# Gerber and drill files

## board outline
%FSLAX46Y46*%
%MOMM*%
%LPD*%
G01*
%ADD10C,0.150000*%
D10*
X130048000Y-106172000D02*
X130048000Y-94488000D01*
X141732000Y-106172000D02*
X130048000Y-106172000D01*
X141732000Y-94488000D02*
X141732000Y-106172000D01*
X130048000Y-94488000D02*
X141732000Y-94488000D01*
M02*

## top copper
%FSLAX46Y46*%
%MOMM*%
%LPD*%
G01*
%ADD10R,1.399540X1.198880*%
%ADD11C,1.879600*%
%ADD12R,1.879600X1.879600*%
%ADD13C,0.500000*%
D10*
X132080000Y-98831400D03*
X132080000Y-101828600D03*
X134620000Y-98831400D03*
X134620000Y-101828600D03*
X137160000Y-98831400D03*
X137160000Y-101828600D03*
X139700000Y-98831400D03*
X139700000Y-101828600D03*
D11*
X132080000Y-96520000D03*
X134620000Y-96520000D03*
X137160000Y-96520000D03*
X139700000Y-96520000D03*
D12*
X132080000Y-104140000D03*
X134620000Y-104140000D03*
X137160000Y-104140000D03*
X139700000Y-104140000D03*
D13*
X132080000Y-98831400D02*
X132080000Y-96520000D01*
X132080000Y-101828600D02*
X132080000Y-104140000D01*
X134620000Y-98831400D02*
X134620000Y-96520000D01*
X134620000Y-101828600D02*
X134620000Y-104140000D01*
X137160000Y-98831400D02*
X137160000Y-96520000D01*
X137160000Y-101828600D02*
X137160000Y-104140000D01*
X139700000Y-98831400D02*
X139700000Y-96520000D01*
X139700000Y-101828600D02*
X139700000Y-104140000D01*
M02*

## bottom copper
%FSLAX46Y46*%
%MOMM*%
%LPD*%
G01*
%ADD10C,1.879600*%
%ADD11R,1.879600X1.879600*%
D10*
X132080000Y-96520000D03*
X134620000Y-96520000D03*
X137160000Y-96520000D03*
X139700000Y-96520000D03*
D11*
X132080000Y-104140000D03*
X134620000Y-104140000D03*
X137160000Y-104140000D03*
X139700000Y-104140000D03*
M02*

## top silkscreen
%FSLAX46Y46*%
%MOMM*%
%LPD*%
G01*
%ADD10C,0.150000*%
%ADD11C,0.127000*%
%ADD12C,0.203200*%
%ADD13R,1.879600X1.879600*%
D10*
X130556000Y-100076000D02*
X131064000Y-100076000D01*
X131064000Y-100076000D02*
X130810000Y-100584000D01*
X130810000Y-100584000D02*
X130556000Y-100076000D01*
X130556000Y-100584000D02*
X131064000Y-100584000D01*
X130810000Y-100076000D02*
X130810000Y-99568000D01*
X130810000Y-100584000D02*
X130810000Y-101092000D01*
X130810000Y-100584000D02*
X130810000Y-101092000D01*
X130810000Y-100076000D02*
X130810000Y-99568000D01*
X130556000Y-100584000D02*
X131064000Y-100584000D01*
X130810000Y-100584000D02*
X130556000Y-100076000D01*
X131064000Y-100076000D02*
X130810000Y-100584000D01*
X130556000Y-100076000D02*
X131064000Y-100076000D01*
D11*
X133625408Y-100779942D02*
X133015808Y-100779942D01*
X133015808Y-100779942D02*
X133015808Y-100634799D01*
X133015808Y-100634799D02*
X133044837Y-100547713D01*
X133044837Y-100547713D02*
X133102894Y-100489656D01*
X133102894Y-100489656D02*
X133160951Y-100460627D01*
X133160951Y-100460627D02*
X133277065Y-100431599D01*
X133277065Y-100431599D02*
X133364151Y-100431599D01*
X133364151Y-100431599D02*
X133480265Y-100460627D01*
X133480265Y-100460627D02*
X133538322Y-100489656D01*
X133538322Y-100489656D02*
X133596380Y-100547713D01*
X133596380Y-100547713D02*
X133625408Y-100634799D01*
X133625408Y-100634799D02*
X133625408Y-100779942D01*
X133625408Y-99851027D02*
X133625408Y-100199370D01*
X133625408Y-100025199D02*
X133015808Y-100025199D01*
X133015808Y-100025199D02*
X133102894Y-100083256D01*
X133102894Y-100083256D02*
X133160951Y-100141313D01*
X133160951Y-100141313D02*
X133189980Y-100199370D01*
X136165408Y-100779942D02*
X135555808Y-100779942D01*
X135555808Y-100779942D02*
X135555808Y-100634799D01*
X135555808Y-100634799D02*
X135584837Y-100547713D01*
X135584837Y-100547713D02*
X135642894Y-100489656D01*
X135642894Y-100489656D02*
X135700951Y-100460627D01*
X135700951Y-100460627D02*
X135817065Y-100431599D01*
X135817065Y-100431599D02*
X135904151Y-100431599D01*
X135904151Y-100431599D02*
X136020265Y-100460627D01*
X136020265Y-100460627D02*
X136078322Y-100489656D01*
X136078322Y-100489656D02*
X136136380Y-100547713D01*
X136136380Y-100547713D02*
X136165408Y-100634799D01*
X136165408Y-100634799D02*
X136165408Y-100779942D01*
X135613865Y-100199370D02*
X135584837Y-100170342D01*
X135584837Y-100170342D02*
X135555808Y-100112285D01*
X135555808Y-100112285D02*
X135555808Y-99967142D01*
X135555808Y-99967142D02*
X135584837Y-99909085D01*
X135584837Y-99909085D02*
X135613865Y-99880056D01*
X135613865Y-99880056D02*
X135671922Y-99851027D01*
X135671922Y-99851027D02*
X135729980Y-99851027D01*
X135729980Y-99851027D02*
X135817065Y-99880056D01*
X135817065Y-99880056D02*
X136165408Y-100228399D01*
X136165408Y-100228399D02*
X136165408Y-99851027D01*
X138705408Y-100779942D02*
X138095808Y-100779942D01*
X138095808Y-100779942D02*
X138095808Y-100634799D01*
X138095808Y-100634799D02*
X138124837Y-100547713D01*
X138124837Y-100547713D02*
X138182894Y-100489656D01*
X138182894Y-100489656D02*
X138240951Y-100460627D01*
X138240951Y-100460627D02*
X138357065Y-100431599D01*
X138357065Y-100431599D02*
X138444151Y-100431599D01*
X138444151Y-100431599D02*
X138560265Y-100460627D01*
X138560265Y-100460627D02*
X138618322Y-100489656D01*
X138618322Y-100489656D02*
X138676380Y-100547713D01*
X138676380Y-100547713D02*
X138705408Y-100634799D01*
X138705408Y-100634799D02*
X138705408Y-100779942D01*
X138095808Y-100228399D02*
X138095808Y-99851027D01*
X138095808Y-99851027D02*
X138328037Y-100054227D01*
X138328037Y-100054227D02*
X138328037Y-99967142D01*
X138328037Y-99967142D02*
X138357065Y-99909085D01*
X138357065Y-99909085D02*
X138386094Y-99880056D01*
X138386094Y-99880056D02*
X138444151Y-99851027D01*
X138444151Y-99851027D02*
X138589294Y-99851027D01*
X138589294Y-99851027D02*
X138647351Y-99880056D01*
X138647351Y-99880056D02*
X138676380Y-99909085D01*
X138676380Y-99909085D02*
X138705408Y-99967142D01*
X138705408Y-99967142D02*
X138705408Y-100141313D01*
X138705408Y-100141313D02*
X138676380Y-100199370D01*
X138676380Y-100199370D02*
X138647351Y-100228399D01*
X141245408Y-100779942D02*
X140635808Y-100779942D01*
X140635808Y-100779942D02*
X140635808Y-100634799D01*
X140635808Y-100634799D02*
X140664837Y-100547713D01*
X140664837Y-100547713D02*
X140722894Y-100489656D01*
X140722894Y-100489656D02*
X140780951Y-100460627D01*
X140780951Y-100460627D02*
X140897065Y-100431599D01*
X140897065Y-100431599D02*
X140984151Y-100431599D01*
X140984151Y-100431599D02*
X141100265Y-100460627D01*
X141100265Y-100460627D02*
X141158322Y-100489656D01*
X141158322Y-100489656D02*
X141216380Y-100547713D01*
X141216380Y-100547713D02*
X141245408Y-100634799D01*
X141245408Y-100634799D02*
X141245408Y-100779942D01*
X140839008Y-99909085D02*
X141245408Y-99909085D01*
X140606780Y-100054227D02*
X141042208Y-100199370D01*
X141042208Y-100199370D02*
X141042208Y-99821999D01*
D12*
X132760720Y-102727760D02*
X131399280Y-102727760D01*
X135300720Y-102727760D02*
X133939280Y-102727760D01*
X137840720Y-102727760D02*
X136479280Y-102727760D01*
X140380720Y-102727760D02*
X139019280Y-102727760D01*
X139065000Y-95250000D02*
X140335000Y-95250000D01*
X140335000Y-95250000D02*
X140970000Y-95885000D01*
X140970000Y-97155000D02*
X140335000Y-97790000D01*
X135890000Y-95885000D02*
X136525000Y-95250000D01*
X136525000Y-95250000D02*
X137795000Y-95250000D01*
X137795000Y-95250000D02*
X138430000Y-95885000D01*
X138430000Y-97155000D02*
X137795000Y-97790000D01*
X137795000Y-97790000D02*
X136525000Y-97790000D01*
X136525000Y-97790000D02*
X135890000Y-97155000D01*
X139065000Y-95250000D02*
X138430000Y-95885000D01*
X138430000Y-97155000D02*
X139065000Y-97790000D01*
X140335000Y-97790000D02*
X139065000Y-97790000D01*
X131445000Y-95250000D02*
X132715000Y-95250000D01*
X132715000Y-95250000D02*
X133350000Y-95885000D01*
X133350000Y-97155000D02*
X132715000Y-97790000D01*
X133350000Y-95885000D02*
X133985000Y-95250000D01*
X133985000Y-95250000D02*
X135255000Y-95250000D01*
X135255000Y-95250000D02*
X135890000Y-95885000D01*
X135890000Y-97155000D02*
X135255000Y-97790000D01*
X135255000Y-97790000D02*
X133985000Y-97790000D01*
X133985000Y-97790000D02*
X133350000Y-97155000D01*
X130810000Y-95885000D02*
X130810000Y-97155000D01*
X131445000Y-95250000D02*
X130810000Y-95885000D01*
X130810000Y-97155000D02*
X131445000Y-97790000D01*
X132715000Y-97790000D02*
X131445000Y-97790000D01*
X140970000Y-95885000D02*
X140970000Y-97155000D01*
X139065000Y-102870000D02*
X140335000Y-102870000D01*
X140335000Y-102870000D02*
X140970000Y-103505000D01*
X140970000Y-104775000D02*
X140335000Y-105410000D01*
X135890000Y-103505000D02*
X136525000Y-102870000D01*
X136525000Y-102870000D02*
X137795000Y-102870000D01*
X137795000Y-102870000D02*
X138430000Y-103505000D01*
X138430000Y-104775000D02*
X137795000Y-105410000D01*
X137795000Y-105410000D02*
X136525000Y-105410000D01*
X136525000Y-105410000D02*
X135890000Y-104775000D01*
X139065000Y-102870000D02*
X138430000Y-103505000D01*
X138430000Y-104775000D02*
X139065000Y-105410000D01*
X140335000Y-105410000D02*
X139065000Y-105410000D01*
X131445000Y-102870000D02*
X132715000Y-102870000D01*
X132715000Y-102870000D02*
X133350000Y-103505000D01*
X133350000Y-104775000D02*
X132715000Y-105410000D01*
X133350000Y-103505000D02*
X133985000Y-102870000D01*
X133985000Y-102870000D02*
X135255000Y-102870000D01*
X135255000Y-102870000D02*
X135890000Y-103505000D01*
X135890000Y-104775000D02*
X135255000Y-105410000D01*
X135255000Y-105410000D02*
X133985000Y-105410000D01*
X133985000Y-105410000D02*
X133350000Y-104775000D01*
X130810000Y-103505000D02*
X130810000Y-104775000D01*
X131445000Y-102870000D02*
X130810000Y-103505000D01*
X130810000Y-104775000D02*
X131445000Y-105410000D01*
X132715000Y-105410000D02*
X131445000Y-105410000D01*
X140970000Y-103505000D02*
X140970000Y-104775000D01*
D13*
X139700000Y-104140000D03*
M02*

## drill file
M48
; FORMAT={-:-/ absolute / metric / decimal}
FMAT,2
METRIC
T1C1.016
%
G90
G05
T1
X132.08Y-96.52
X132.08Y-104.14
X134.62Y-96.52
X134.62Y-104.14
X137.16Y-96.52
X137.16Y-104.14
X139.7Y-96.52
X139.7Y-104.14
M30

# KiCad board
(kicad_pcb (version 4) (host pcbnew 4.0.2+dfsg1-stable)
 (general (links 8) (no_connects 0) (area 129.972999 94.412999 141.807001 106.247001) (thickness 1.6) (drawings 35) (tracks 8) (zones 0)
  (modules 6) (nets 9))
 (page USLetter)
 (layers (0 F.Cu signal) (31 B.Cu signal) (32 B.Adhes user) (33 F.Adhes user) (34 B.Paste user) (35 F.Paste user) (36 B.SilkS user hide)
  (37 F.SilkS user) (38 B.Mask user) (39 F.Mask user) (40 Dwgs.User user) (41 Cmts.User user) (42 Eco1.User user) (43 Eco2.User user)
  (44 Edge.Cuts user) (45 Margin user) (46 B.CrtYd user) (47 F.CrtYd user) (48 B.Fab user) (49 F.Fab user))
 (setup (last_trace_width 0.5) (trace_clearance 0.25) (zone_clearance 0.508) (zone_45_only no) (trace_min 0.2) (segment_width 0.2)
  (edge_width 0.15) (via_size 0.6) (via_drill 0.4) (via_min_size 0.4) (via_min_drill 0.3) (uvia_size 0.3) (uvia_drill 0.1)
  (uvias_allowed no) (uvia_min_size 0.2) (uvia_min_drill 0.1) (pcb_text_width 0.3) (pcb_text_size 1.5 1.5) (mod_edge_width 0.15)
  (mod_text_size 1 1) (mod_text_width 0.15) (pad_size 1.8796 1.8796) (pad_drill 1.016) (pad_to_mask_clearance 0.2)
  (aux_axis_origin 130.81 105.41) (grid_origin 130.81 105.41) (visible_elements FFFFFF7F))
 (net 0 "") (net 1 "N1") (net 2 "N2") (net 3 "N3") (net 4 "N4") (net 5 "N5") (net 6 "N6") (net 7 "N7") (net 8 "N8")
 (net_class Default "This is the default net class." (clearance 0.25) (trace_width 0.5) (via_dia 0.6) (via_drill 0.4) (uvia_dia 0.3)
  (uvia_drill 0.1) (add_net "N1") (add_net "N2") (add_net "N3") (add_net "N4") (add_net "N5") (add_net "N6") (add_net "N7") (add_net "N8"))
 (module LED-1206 (layer F.Cu) (at 132.08 100.33 270)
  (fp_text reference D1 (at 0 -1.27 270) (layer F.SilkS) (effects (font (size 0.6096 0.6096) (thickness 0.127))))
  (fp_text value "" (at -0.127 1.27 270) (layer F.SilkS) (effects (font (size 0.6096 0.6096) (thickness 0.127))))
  (fp_line (start 2.39776 -0.68072) (end 2.39776 0.68072) (layer F.SilkS) (width 0.2032))
  (pad A smd rect (at -1.4986 0 270) (size 1.19888 1.39954) (layers F.Cu F.Paste F.Mask) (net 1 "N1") (solder_mask_margin 0.1016))
  (pad C smd rect (at 1.4986 0 270) (size 1.19888 1.39954) (layers F.Cu F.Paste F.Mask) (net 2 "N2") (solder_mask_margin 0.1016)))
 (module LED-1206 (layer F.Cu) (at 134.62 100.33 270)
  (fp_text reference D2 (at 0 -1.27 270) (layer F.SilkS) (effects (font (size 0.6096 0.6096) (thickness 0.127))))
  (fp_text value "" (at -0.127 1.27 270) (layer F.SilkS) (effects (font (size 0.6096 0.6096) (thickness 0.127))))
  (fp_line (start 2.39776 -0.68072) (end 2.39776 0.68072) (layer F.SilkS) (width 0.2032))
  (pad A smd rect (at -1.4986 0 270) (size 1.19888 1.39954) (layers F.Cu F.Paste F.Mask) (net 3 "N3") (solder_mask_margin 0.1016))
  (pad C smd rect (at 1.4986 0 270) (size 1.19888 1.39954) (layers F.Cu F.Paste F.Mask) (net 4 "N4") (solder_mask_margin 0.1016)))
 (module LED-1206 (layer F.Cu) (at 137.16 100.33 270)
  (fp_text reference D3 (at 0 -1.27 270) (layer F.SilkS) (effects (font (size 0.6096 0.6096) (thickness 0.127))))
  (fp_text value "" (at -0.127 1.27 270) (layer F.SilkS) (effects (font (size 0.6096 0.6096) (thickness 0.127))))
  (fp_line (start 2.39776 -0.68072) (end 2.39776 0.68072) (layer F.SilkS) (width 0.2032))
  (pad A smd rect (at -1.4986 0 270) (size 1.19888 1.39954) (layers F.Cu F.Paste F.Mask) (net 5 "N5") (solder_mask_margin 0.1016))
  (pad C smd rect (at 1.4986 0 270) (size 1.19888 1.39954) (layers F.Cu F.Paste F.Mask) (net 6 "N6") (solder_mask_margin 0.1016)))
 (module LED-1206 (layer F.Cu) (at 139.7 100.33 270)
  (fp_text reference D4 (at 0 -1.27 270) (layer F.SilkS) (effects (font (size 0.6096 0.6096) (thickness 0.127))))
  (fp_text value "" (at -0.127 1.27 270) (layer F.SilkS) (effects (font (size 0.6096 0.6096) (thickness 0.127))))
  (fp_line (start 2.39776 -0.68072) (end 2.39776 0.68072) (layer F.SilkS) (width 0.2032))
  (pad A smd rect (at -1.4986 0 270) (size 1.19888 1.39954) (layers F.Cu F.Paste F.Mask) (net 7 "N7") (solder_mask_margin 0.1016))
  (pad C smd rect (at 1.4986 0 270) (size 1.19888 1.39954) (layers F.Cu F.Paste F.Mask) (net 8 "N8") (solder_mask_margin 0.1016)))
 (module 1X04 (layer F.Cu) (at 132.08 96.52)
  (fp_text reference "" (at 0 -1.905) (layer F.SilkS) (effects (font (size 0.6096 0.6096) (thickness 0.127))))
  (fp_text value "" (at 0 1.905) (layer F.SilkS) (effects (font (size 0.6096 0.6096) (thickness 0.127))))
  (fp_line (start 6.985 -1.27) (end 8.255 -1.27) (layer F.SilkS) (width 0.2032))
  (fp_line (start 8.255 -1.27) (end 8.89 -0.635) (layer F.SilkS) (width 0.2032))
  (fp_line (start 8.89 0.635) (end 8.255 1.27) (layer F.SilkS) (width 0.2032))
  (fp_line (start 3.81 -0.635) (end 4.445 -1.27) (layer F.SilkS) (width 0.2032))
  (fp_line (start 4.445 -1.27) (end 5.715 -1.27) (layer F.SilkS) (width 0.2032))
  (fp_line (start 5.715 -1.27) (end 6.35 -0.635) (layer F.SilkS) (width 0.2032))
  (fp_line (start 6.35 0.635) (end 5.715 1.27) (layer F.SilkS) (width 0.2032))
  (fp_line (start 5.715 1.27) (end 4.445 1.27) (layer F.SilkS) (width 0.2032))
  (fp_line (start 4.445 1.27) (end 3.81 0.635) (layer F.SilkS) (width 0.2032))
  (fp_line (start 6.985 -1.27) (end 6.35 -0.635) (layer F.SilkS) (width 0.2032))
  (fp_line (start 6.35 0.635) (end 6.985 1.27) (layer F.SilkS) (width 0.2032))
  (fp_line (start 8.255 1.27) (end 6.985 1.27) (layer F.SilkS) (width 0.2032))
  (fp_line (start -0.635 -1.27) (end 0.635 -1.27) (layer F.SilkS) (width 0.2032))
  (fp_line (start 0.635 -1.27) (end 1.27 -0.635) (layer F.SilkS) (width 0.2032))
  (fp_line (start 1.27 0.635) (end 0.635 1.27) (layer F.SilkS) (width 0.2032))
  (fp_line (start 1.27 -0.635) (end 1.905 -1.27) (layer F.SilkS) (width 0.2032))
  (fp_line (start 1.905 -1.27) (end 3.175 -1.27) (layer F.SilkS) (width 0.2032))
  (fp_line (start 3.175 -1.27) (end 3.81 -0.635) (layer F.SilkS) (width 0.2032))
  (fp_line (start 3.81 0.635) (end 3.175 1.27) (layer F.SilkS) (width 0.2032))
  (fp_line (start 3.175 1.27) (end 1.905 1.27) (layer F.SilkS) (width 0.2032))
  (fp_line (start 1.905 1.27) (end 1.27 0.635) (layer F.SilkS) (width 0.2032))
  (fp_line (start -1.27 -0.635) (end -1.27 0.635) (layer F.SilkS) (width 0.2032))
  (fp_line (start -0.635 -1.27) (end -1.27 -0.635) (layer F.SilkS) (width 0.2032))
  (fp_line (start -1.27 0.635) (end -0.635 1.27) (layer F.SilkS) (width 0.2032))
  (fp_line (start 0.635 1.27) (end -0.635 1.27) (layer F.SilkS) (width 0.2032))
  (fp_line (start 8.89 -0.635) (end 8.89 0.635) (layer F.SilkS) (width 0.2032))
  (pad 1 thru_hole circle (at 0 0) (size 1.8796 1.8796) (drill 1.016) (layers *.Cu *.Mask) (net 1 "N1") (solder_mask_margin 0.1016))
  (pad 2 thru_hole circle (at 2.54 0) (size 1.8796 1.8796) (drill 1.016) (layers *.Cu *.Mask) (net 3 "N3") (solder_mask_margin 0.1016))
  (pad 3 thru_hole circle (at 5.08 0) (size 1.8796 1.8796) (drill 1.016) (layers *.Cu *.Mask) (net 5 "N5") (solder_mask_margin 0.1016))
  (pad 4 thru_hole circle (at 7.62 0) (size 1.8796 1.8796) (drill 1.016) (layers *.Cu *.Mask) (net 7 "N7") (solder_mask_margin 0.1016)))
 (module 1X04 (layer F.Cu) (at 132.08 104.14)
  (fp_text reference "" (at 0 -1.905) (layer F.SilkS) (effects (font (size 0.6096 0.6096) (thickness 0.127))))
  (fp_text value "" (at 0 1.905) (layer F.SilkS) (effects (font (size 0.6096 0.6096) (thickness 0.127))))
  (fp_line (start 6.985 -1.27) (end 8.255 -1.27) (layer F.SilkS) (width 0.2032))
  (fp_line (start 8.255 -1.27) (end 8.89 -0.635) (layer F.SilkS) (width 0.2032))
  (fp_line (start 8.89 0.635) (end 8.255 1.27) (layer F.SilkS) (width 0.2032))
  (fp_line (start 3.81 -0.635) (end 4.445 -1.27) (layer F.SilkS) (width 0.2032))
  (fp_line (start 4.445 -1.27) (end 5.715 -1.27) (layer F.SilkS) (width 0.2032))
  (fp_line (start 5.715 -1.27) (end 6.35 -0.635) (layer F.SilkS) (width 0.2032))
  (fp_line (start 6.35 0.635) (end 5.715 1.27) (layer F.SilkS) (width 0.2032))
  (fp_line (start 5.715 1.27) (end 4.445 1.27) (layer F.SilkS) (width 0.2032))
  (fp_line (start 4.445 1.27) (end 3.81 0.635) (layer F.SilkS) (width 0.2032))
  (fp_line (start 6.985 -1.27) (end 6.35 -0.635) (layer F.SilkS) (width 0.2032))
  (fp_line (start 6.35 0.635) (end 6.985 1.27) (layer F.SilkS) (width 0.2032))
  (fp_line (start 8.255 1.27) (end 6.985 1.27) (layer F.SilkS) (width 0.2032))
  (fp_line (start -0.635 -1.27) (end 0.635 -1.27) (layer F.SilkS) (width 0.2032))
  (fp_line (start 0.635 -1.27) (end 1.27 -0.635) (layer F.SilkS) (width 0.2032))
  (fp_line (start 1.27 0.635) (end 0.635 1.27) (layer F.SilkS) (width 0.2032))
  (fp_line (start 1.27 -0.635) (end 1.905 -1.27) (layer F.SilkS) (width 0.2032))
  (fp_line (start 1.905 -1.27) (end 3.175 -1.27) (layer F.SilkS) (width 0.2032))
  (fp_line (start 3.175 -1.27) (end 3.81 -0.635) (layer F.SilkS) (width 0.2032))
  (fp_line (start 3.81 0.635) (end 3.175 1.27) (layer F.SilkS) (width 0.2032))
  (fp_line (start 3.175 1.27) (end 1.905 1.27) (layer F.SilkS) (width 0.2032))
  (fp_line (start 1.905 1.27) (end 1.27 0.635) (layer F.SilkS) (width 0.2032))
  (fp_line (start -1.27 -0.635) (end -1.27 0.635) (layer F.SilkS) (width 0.2032))
  (fp_line (start -0.635 -1.27) (end -1.27 -0.635) (layer F.SilkS) (width 0.2032))
  (fp_line (start -1.27 0.635) (end -0.635 1.27) (layer F.SilkS) (width 0.2032))
  (fp_line (start 0.635 1.27) (end -0.635 1.27) (layer F.SilkS) (width 0.2032))
  (fp_line (start 8.89 -0.635) (end 8.89 0.635) (layer F.SilkS) (width 0.2032))
  (pad 1 thru_hole rect (at 0 0) (size 1.8796 1.8796) (drill 1.016) (layers *.Cu *.Mask) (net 2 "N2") (solder_mask_margin 0.1016))
  (pad 2 thru_hole rect (at 2.54 0) (size 1.8796 1.8796) (drill 1.016) (layers *.Cu *.Mask) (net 4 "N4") (solder_mask_margin 0.1016))
  (pad 3 thru_hole rect (at 5.08 0) (size 1.8796 1.8796) (drill 1.016) (layers *.Cu *.Mask) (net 6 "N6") (solder_mask_margin 0.1016))
  (pad 4 thru_hole rect (at 7.62 0) (size 1.8796 1.8796) (drill 1.016) (layers *.Cu *.Mask F.SilkS) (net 8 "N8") (solder_mask_margin 0.1016)))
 (gr_line (start 130.556 100.076) (end 131.064 100.076) (angle 90) (layer F.SilkS) (width 0.15))
 (gr_line (start 131.064 100.076) (end 130.81 100.584) (angle 90) (layer F.SilkS) (width 0.15))
 (gr_line (start 130.81 100.584) (end 130.556 100.076) (angle 90) (layer F.SilkS) (width 0.15))
 (gr_line (start 130.556 100.584) (end 131.064 100.584) (angle 90) (layer F.SilkS) (width 0.15))
 (gr_line (start 130.81 100.076) (end 130.81 99.568) (angle 90) (layer F.SilkS) (width 0.15))
 (gr_line (start 130.81 100.584) (end 130.81 101.092) (angle 90) (layer F.SilkS) (width 0.15))
 (gr_line (start 130.81 100.584) (end 130.81 101.092) (angle 90) (layer F.SilkS) (width 0.15))
 (gr_line (start 130.81 100.076) (end 130.81 99.568) (angle 90) (layer F.SilkS) (width 0.15))
 (gr_line (start 130.556 100.584) (end 131.064 100.584) (angle 90) (layer F.SilkS) (width 0.15))
 (gr_line (start 130.81 100.584) (end 130.556 100.076) (angle 90) (layer F.SilkS) (width 0.15))
 (gr_line (start 131.064 100.076) (end 130.81 100.584) (angle 90) (layer F.SilkS) (width 0.15))
 (gr_line (start 130.556 100.076) (end 131.064 100.076) (angle 90) (layer F.SilkS) (width 0.15))
 (gr_line (start 130.048 106.172) (end 130.048 94.488) (angle 90) (layer Edge.Cuts) (width 0.15))
 (gr_line (start 141.732 106.172) (end 130.048 106.172) (angle 90) (layer Edge.Cuts) (width 0.15))
 (gr_line (start 141.732 94.488) (end 141.732 106.172) (angle 90) (layer Edge.Cuts) (width 0.15))
 (gr_line (start 130.048 94.488) (end 141.732 94.488) (angle 90) (layer Edge.Cuts) (width 0.15))
 (segment (start 132.08 98.8314) (end 132.08 96.52) (width 0.5) (layer F.Cu) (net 1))
 (segment (start 132.08 101.8286) (end 132.08 104.14) (width 0.5) (layer F.Cu) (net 2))
 (segment (start 134.62 98.8314) (end 134.62 96.52) (width 0.5) (layer F.Cu) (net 3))
 (segment (start 134.62 101.8286) (end 134.62 104.14) (width 0.5) (layer F.Cu) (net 4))
 (segment (start 137.16 98.8314) (end 137.16 96.52) (width 0.5) (layer F.Cu) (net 5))
 (segment (start 137.16 101.8286) (end 137.16 104.14) (width 0.5) (layer F.Cu) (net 6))
 (segment (start 139.7 98.8314) (end 139.7 96.52) (width 0.5) (layer F.Cu) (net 7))
 (segment (start 139.7 101.8286) (end 139.7 104.14) (width 0.5) (layer F.Cu) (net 8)))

